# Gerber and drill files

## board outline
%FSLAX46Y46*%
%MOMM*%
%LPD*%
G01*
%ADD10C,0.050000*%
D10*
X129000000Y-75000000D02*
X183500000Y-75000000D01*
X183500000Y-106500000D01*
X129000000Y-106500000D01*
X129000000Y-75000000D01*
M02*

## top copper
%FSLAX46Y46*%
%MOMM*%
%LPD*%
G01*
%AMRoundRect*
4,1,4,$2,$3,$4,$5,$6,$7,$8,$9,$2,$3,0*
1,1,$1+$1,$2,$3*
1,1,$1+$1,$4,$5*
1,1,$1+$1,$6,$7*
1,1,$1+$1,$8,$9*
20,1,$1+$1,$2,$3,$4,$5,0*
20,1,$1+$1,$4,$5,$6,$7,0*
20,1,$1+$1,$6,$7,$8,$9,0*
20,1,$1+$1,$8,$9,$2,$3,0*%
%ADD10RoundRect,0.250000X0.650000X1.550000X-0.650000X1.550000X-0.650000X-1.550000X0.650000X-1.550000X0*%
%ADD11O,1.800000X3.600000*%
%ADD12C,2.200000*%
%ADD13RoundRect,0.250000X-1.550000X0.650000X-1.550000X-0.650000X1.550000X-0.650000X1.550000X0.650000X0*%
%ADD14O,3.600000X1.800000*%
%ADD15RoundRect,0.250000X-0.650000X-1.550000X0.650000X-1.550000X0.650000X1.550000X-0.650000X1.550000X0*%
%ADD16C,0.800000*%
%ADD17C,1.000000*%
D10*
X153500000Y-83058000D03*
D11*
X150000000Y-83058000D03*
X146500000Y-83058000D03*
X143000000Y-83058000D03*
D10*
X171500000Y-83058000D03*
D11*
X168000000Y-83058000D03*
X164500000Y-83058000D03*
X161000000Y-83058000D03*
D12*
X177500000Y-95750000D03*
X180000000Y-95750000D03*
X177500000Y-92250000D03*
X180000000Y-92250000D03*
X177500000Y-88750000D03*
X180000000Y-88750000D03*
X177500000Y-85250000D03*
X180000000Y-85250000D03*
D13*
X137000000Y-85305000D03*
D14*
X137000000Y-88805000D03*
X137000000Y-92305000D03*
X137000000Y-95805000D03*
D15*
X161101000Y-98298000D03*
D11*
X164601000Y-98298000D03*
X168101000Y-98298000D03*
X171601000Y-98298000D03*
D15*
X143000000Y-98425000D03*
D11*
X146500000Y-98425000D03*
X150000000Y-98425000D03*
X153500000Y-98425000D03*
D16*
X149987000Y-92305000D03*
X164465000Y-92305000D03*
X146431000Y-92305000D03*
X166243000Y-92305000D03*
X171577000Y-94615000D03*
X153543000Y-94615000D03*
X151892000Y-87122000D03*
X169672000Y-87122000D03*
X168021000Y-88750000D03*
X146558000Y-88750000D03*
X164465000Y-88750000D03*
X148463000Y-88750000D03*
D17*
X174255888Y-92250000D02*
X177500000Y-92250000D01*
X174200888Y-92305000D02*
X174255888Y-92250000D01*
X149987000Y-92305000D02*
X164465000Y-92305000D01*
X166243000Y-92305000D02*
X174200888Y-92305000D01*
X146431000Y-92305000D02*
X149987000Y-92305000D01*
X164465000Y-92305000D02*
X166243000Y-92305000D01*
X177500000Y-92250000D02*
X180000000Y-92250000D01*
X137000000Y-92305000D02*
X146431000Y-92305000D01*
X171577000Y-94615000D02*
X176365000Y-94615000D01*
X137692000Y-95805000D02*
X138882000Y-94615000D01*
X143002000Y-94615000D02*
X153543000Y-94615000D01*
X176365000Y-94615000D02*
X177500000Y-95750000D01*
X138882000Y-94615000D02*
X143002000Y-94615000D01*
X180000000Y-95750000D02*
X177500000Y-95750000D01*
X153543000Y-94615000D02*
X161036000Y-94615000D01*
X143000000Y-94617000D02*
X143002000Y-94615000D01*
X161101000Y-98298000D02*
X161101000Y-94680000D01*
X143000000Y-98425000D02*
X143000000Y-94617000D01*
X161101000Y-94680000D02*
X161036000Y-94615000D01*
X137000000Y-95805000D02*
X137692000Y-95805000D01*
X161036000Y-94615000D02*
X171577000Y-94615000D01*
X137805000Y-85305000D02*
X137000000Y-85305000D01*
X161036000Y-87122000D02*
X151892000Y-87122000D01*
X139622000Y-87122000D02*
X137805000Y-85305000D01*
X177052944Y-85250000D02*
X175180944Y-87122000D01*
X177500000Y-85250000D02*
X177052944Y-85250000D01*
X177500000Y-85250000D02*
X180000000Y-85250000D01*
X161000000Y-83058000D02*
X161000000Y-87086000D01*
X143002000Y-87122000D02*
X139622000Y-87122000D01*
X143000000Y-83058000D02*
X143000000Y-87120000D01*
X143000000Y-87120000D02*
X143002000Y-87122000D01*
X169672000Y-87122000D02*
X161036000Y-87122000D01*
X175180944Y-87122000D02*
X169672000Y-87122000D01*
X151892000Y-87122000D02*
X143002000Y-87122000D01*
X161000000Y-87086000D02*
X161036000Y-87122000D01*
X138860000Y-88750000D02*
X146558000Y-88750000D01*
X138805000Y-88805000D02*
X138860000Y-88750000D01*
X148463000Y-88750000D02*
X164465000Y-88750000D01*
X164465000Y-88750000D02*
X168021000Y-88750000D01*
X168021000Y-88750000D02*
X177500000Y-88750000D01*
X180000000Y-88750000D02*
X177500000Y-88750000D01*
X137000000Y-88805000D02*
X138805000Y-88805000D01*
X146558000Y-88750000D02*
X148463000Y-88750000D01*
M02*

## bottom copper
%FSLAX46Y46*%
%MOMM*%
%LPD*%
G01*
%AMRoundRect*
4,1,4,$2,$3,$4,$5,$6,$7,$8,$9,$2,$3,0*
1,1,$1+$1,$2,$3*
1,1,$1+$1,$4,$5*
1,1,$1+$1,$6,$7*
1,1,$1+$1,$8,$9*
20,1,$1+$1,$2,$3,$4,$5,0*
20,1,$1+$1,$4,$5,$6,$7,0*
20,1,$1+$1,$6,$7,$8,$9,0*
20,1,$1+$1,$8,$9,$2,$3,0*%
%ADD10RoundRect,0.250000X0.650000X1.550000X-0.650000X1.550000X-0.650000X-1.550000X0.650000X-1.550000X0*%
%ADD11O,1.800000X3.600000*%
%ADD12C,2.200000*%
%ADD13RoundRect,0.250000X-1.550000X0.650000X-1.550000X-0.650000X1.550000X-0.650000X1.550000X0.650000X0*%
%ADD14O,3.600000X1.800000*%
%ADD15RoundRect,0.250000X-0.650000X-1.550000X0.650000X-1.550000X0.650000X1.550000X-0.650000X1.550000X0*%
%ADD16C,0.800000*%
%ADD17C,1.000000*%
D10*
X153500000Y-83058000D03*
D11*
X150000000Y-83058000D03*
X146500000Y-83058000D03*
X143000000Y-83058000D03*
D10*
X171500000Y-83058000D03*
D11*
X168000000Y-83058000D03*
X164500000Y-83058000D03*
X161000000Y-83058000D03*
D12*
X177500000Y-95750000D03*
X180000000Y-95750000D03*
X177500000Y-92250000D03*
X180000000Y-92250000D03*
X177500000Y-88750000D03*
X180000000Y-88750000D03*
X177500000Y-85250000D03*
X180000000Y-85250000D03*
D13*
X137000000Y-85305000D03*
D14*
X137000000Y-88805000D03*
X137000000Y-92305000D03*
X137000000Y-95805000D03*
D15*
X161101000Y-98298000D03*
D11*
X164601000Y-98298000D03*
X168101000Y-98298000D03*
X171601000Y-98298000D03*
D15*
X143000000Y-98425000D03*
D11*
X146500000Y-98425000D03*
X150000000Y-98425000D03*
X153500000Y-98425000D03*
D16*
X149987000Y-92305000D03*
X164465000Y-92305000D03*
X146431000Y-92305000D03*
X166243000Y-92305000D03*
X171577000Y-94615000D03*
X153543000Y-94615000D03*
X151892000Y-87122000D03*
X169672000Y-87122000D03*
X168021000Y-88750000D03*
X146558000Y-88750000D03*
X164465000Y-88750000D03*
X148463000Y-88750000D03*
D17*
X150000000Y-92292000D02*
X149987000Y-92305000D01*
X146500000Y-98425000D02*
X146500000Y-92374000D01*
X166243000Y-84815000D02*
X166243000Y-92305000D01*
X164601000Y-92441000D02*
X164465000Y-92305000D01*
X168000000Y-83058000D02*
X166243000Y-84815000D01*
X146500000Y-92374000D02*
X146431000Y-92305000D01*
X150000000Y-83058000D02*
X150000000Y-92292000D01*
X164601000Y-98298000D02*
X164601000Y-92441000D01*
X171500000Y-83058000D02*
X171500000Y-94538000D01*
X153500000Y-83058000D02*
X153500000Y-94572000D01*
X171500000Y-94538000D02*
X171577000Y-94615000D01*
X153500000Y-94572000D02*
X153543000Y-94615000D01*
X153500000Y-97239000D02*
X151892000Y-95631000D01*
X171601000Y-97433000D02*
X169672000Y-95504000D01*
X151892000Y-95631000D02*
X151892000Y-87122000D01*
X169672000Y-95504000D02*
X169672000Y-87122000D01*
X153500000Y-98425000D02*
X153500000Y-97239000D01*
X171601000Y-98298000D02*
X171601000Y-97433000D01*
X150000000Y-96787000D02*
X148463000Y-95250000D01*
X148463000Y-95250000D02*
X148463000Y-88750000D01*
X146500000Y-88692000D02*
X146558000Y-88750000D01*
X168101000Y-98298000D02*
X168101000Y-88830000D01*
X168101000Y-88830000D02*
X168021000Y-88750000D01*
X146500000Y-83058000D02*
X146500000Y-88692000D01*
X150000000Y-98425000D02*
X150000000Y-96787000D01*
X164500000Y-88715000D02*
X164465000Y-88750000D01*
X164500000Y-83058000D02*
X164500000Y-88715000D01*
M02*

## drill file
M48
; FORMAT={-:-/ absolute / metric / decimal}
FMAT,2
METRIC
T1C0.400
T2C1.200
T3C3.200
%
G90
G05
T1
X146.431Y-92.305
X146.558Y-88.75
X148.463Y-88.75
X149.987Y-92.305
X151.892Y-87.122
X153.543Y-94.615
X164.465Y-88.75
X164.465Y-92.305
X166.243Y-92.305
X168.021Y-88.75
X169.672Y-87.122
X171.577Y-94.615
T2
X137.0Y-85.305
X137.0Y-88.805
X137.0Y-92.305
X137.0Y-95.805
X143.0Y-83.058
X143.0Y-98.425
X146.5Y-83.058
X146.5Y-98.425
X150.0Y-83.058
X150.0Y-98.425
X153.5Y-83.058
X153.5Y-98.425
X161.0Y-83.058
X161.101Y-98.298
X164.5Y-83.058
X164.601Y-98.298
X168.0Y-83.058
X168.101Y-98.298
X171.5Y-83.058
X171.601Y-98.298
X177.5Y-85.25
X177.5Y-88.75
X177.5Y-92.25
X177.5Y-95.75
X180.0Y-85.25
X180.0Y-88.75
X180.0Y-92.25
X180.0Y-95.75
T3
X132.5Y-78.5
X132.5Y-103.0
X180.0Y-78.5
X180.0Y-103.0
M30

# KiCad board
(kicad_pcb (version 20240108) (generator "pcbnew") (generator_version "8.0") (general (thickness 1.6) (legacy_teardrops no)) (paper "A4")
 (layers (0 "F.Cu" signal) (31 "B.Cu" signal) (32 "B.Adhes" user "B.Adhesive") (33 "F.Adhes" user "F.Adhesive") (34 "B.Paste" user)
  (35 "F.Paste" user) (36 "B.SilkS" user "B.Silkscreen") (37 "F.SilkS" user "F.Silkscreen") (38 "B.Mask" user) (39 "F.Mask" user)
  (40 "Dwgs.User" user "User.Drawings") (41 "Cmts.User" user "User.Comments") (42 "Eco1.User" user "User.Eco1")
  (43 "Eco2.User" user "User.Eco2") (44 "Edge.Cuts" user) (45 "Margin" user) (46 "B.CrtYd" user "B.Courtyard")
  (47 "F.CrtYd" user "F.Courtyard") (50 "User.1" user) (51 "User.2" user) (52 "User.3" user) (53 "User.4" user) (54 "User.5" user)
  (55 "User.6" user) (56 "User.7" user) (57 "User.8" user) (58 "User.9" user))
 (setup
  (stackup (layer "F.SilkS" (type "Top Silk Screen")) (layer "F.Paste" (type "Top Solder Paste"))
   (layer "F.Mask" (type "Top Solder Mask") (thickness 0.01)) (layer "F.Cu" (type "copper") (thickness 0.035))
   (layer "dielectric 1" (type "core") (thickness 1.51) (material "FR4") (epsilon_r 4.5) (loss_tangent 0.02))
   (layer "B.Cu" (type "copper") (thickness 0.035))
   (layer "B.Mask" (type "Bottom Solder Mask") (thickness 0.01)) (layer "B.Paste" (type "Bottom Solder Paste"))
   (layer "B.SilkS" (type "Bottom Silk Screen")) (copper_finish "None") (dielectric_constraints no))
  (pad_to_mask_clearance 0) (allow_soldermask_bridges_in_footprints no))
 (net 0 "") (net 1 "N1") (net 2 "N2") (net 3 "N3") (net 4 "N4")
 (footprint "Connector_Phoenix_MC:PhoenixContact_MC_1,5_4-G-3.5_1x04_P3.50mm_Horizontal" (layer "F.Cu") (at 153.5 83.058 180)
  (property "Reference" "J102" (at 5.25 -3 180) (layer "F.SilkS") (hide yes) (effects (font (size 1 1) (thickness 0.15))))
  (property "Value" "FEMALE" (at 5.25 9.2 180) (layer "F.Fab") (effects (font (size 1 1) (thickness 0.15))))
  (pad "1" thru_hole roundrect (at 0 0 180) (size 1.8 3.6) (drill 1.2) (layers "*.Cu" "*.Mask") (remove_unused_layers no)
   (roundrect_rratio 0.138889) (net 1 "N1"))
  (pad "2" thru_hole oval (at 3.5 0 180) (size 1.8 3.6) (drill 1.2) (layers "*.Cu" "*.Mask") (remove_unused_layers no) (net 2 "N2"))
  (pad "3" thru_hole oval (at 7 0 180) (size 1.8 3.6) (drill 1.2) (layers "*.Cu" "*.Mask") (remove_unused_layers no) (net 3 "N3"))
  (pad "4" thru_hole oval (at 10.5 0 180) (size 1.8 3.6) (drill 1.2) (layers "*.Cu" "*.Mask") (remove_unused_layers no) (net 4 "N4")))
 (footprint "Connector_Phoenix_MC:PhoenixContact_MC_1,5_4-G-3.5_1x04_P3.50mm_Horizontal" (layer "F.Cu") (at 171.5 83.058 180)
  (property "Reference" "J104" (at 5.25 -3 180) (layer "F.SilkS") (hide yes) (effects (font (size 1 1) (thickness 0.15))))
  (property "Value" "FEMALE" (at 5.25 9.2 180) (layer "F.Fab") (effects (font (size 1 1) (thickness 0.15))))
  (pad "1" thru_hole roundrect (at 0 0 180) (size 1.8 3.6) (drill 1.2) (layers "*.Cu" "*.Mask") (remove_unused_layers no)
   (roundrect_rratio 0.138889) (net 1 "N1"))
  (pad "2" thru_hole oval (at 3.5 0 180) (size 1.8 3.6) (drill 1.2) (layers "*.Cu" "*.Mask") (remove_unused_layers no) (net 2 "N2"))
  (pad "3" thru_hole oval (at 7 0 180) (size 1.8 3.6) (drill 1.2) (layers "*.Cu" "*.Mask") (remove_unused_layers no) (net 3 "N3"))
  (pad "4" thru_hole oval (at 10.5 0 180) (size 1.8 3.6) (drill 1.2) (layers "*.Cu" "*.Mask") (remove_unused_layers no) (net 4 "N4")))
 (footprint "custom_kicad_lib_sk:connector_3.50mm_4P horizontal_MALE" (layer "F.Cu") (at 177.5 90.5 90)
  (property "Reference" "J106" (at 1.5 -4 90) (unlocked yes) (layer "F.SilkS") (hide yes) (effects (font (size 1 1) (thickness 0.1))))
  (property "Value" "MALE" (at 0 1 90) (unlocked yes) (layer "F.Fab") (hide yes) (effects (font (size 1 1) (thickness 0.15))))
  (pad "1" thru_hole circle (at -5.25 0 90) (size 2.2 2.2) (drill 1.2) (layers "*.Cu" "*.Mask") (remove_unused_layers no) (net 1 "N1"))
  (pad "1" thru_hole circle (at -5.25 2.5 90) (size 2.2 2.2) (drill 1.2) (layers "*.Cu" "*.Mask") (remove_unused_layers no) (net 1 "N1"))
  (pad "2" thru_hole circle (at -1.75 0 90) (size 2.2 2.2) (drill 1.2) (layers "*.Cu" "*.Mask") (remove_unused_layers no) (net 2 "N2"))
  (pad "2" thru_hole circle (at -1.75 2.5 90) (size 2.2 2.2) (drill 1.2) (layers "*.Cu" "*.Mask") (remove_unused_layers no) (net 2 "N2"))
  (pad "3" thru_hole circle (at 1.75 0 90) (size 2.2 2.2) (drill 1.2) (layers "*.Cu" "*.Mask") (remove_unused_layers no) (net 3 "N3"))
  (pad "3" thru_hole circle (at 1.75 2.5 90) (size 2.2 2.2) (drill 1.2) (layers "*.Cu" "*.Mask") (remove_unused_layers no) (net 3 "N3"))
  (pad "4" thru_hole circle (at 5.25 0 90) (size 2.2 2.2) (drill 1.2) (layers "*.Cu" "*.Mask") (remove_unused_layers no) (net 4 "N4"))
  (pad "4" thru_hole circle (at 5.25 2.5 90) (size 2.2 2.2) (drill 1.2) (layers "*.Cu" "*.Mask") (remove_unused_layers no) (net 4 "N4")))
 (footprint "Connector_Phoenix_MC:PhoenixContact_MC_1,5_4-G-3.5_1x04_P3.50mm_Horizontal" (layer "F.Cu") (at 137 85.305 -90)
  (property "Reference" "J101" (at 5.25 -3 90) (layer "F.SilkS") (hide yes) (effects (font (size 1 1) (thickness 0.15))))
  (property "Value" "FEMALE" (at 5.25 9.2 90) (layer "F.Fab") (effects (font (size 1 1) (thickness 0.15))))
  (pad "1" thru_hole roundrect (at 0 0 270) (size 1.8 3.6) (drill 1.2) (layers "*.Cu" "*.Mask") (remove_unused_layers no)
   (roundrect_rratio 0.138889) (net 4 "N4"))
  (pad "2" thru_hole oval (at 3.5 0 270) (size 1.8 3.6) (drill 1.2) (layers "*.Cu" "*.Mask") (remove_unused_layers no) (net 3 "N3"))
  (pad "3" thru_hole oval (at 7 0 270) (size 1.8 3.6) (drill 1.2) (layers "*.Cu" "*.Mask") (remove_unused_layers no) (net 2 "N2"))
  (pad "4" thru_hole oval (at 10.5 0 270) (size 1.8 3.6) (drill 1.2) (layers "*.Cu" "*.Mask") (remove_unused_layers no) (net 1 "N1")))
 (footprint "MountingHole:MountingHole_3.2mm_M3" (layer "F.Cu") (at 132.5 103)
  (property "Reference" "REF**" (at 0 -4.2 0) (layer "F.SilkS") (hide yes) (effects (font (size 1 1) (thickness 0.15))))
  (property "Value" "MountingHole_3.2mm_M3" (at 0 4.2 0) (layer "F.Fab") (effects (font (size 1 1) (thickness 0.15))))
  (pad "" np_thru_hole circle (at 0 0) (size 3.2 3.2) (drill 3.2) (layers "F&B.Cu" "*.Mask")))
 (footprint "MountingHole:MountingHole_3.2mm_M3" (layer "F.Cu") (at 180 78.5)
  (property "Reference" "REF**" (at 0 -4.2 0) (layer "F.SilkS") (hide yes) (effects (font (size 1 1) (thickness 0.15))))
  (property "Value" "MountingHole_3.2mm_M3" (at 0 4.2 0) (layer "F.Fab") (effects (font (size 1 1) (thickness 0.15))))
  (pad "" np_thru_hole circle (at 0 0) (size 3.2 3.2) (drill 3.2) (layers "F&B.Cu" "*.Mask")))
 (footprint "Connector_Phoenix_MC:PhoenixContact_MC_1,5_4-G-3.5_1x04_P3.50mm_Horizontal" (layer "F.Cu") (at 161.101 98.298)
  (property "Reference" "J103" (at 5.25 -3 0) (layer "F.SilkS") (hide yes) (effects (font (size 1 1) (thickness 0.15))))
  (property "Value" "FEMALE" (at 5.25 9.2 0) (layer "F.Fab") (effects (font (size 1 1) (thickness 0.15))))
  (pad "1" thru_hole roundrect (at 0 0) (size 1.8 3.6) (drill 1.2) (layers "*.Cu" "*.Mask") (remove_unused_layers no)
   (roundrect_rratio 0.138889) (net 1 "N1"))
  (pad "2" thru_hole oval (at 3.5 0) (size 1.8 3.6) (drill 1.2) (layers "*.Cu" "*.Mask") (remove_unused_layers no) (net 2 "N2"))
  (pad "3" thru_hole oval (at 7 0) (size 1.8 3.6) (drill 1.2) (layers "*.Cu" "*.Mask") (remove_unused_layers no) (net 3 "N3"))
  (pad "4" thru_hole oval (at 10.5 0) (size 1.8 3.6) (drill 1.2) (layers "*.Cu" "*.Mask") (remove_unused_layers no) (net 4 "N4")))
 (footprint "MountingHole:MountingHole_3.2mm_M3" (layer "F.Cu") (at 180 103)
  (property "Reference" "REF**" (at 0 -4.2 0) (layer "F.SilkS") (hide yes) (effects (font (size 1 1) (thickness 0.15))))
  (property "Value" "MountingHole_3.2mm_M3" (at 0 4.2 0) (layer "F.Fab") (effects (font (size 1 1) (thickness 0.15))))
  (pad "" np_thru_hole circle (at 0 0) (size 3.2 3.2) (drill 3.2) (layers "F&B.Cu" "*.Mask")))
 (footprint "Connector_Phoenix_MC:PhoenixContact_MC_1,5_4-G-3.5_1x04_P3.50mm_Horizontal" (layer "F.Cu") (at 143 98.425)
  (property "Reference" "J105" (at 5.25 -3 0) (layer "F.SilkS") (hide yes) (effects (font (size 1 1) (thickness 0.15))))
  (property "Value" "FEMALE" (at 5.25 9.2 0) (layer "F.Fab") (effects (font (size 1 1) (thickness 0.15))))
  (pad "1" thru_hole roundrect (at 0 0) (size 1.8 3.6) (drill 1.2) (layers "*.Cu" "*.Mask") (remove_unused_layers no)
   (roundrect_rratio 0.138889) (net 1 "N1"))
  (pad "2" thru_hole oval (at 3.5 0) (size 1.8 3.6) (drill 1.2) (layers "*.Cu" "*.Mask") (remove_unused_layers no) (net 2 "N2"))
  (pad "3" thru_hole oval (at 7 0) (size 1.8 3.6) (drill 1.2) (layers "*.Cu" "*.Mask") (remove_unused_layers no) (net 3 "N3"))
  (pad "4" thru_hole oval (at 10.5 0) (size 1.8 3.6) (drill 1.2) (layers "*.Cu" "*.Mask") (remove_unused_layers no) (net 4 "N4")))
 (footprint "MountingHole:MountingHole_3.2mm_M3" (layer "F.Cu") (at 132.5 78.5)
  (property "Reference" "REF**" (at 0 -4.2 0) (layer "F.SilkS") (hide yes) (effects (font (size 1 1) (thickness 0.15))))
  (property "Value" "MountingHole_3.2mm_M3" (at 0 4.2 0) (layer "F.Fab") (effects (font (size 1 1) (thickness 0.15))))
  (pad "" np_thru_hole circle (at 0 0) (size 3.2 3.2) (drill 3.2) (layers "*.Cu" "*.Mask")))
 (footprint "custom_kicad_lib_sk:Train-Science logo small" (layer "B.Cu") (at 157.099 90.932 180)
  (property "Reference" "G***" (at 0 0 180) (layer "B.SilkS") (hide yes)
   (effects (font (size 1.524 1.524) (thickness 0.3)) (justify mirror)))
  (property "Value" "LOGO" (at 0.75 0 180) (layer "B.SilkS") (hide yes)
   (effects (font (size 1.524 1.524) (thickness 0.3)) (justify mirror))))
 (gr_rect (start 129 75) (end 183.5 106.5) (stroke (width 0.05) (type default)) (fill none) (layer "Edge.Cuts"))
 (segment (start 174.255888 92.25) (end 177.5 92.25) (width 1) (layer "F.Cu") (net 2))
 (segment (start 174.200888 92.305) (end 174.255888 92.25) (width 1) (layer "F.Cu") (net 2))
 (segment (start 149.987 92.305) (end 164.465 92.305) (width 1) (layer "F.Cu") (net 2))
 (segment (start 166.243 92.305) (end 174.200888 92.305) (width 1) (layer "F.Cu") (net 2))
 (segment (start 146.431 92.305) (end 149.987 92.305) (width 1) (layer "F.Cu") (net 2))
 (segment (start 164.465 92.305) (end 166.243 92.305) (width 1) (layer "F.Cu") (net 2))
 (segment (start 177.5 92.25) (end 180 92.25) (width 1) (layer "F.Cu") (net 2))
 (segment (start 137 92.305) (end 146.431 92.305) (width 1) (layer "F.Cu") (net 2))
 (via (at 149.987 92.305) (size 0.8) (drill 0.4) (layers "F.Cu" "B.Cu") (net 2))
 (via (at 164.465 92.305) (size 0.8) (drill 0.4) (layers "F.Cu" "B.Cu") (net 2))
 (via (at 146.431 92.305) (size 0.8) (drill 0.4) (layers "F.Cu" "B.Cu") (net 2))
 (via (at 166.243 92.305) (size 0.8) (drill 0.4) (layers "F.Cu" "B.Cu") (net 2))
 (segment (start 150 92.292) (end 149.987 92.305) (width 1) (layer "B.Cu") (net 2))
 (segment (start 146.5 98.425) (end 146.5 92.374) (width 1) (layer "B.Cu") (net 2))
 (segment (start 166.243 84.815) (end 166.243 92.305) (width 1) (layer "B.Cu") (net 2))
 (segment (start 164.601 92.441) (end 164.465 92.305) (width 1) (layer "B.Cu") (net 2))
 (segment (start 168 83.058) (end 166.243 84.815) (width 1) (layer "B.Cu") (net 2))
 (segment (start 146.5 92.374) (end 146.431 92.305) (width 1) (layer "B.Cu") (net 2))
 (segment (start 150 83.058) (end 150 92.292) (width 1) (layer "B.Cu") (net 2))
 (segment (start 164.601 98.298) (end 164.601 92.441) (width 1) (layer "B.Cu") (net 2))
 (segment (start 171.577 94.615) (end 176.365 94.615) (width 1) (layer "F.Cu") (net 1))
 (segment (start 137.692 95.805) (end 138.882 94.615) (width 1) (layer "F.Cu") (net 1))
 (segment (start 143.002 94.615) (end 153.543 94.615) (width 1) (layer "F.Cu") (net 1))
 (segment (start 176.365 94.615) (end 177.5 95.75) (width 1) (layer "F.Cu") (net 1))
 (segment (start 138.882 94.615) (end 143.002 94.615) (width 1) (layer "F.Cu") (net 1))
 (segment (start 180 95.75) (end 177.5 95.75) (width 1) (layer "F.Cu") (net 1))
 (segment (start 153.543 94.615) (end 161.036 94.615) (width 1) (layer "F.Cu") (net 1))
 (segment (start 143 94.617) (end 143.002 94.615) (width 1) (layer "F.Cu") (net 1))
 (segment (start 161.101 98.298) (end 161.101 94.68) (width 1) (layer "F.Cu") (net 1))
 (segment (start 143 98.425) (end 143 94.617) (width 1) (layer "F.Cu") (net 1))
 (segment (start 161.101 94.68) (end 161.036 94.615) (width 1) (layer "F.Cu") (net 1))
 (segment (start 137 95.805) (end 137.692 95.805) (width 1) (layer "F.Cu") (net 1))
 (segment (start 161.036 94.615) (end 171.577 94.615) (width 1) (layer "F.Cu") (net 1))
 (via (at 171.577 94.615) (size 0.8) (drill 0.4) (layers "F.Cu" "B.Cu") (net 1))
 (via (at 153.543 94.615) (size 0.8) (drill 0.4) (layers "F.Cu" "B.Cu") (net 1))
 (segment (start 171.5 83.058) (end 171.5 94.538) (width 1) (layer "B.Cu") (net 1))
 (segment (start 153.5 83.058) (end 153.5 94.572) (width 1) (layer "B.Cu") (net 1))
 (segment (start 171.5 94.538) (end 171.577 94.615) (width 1) (layer "B.Cu") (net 1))
 (segment (start 153.5 94.572) (end 153.543 94.615) (width 1) (layer "B.Cu") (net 1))
 (segment (start 137.805 85.305) (end 137 85.305) (width 1) (layer "F.Cu") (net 4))
 (segment (start 161.036 87.122) (end 151.892 87.122) (width 1) (layer "F.Cu") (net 4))
 (segment (start 139.622 87.122) (end 137.805 85.305) (width 1) (layer "F.Cu") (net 4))
 (segment (start 177.052944 85.25) (end 175.180944 87.122) (width 1) (layer "F.Cu") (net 4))
 (segment (start 177.5 85.25) (end 177.052944 85.25) (width 1) (layer "F.Cu") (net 4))
 (segment (start 177.5 85.25) (end 180 85.25) (width 1) (layer "F.Cu") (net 4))
 (segment (start 161 83.058) (end 161 87.086) (width 1) (layer "F.Cu") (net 4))
 (segment (start 143.002 87.122) (end 139.622 87.122) (width 1) (layer "F.Cu") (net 4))
 (segment (start 143 83.058) (end 143 87.12) (width 1) (layer "F.Cu") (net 4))
 (segment (start 143 87.12) (end 143.002 87.122) (width 1) (layer "F.Cu") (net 4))
 (segment (start 169.672 87.122) (end 161.036 87.122) (width 1) (layer "F.Cu") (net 4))
 (segment (start 175.180944 87.122) (end 169.672 87.122) (width 1) (layer "F.Cu") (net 4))
 (segment (start 151.892 87.122) (end 143.002 87.122) (width 1) (layer "F.Cu") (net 4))
 (segment (start 161 87.086) (end 161.036 87.122) (width 1) (layer "F.Cu") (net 4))
 (via (at 151.892 87.122) (size 0.8) (drill 0.4) (layers "F.Cu" "B.Cu") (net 4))
 (via (at 169.672 87.122) (size 0.8) (drill 0.4) (layers "F.Cu" "B.Cu") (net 4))
 (segment (start 153.5 97.239) (end 151.892 95.631) (width 1) (layer "B.Cu") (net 4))
 (segment (start 171.601 97.433) (end 169.672 95.504) (width 1) (layer "B.Cu") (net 4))
 (segment (start 151.892 95.631) (end 151.892 87.122) (width 1) (layer "B.Cu") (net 4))
 (segment (start 169.672 95.504) (end 169.672 87.122) (width 1) (layer "B.Cu") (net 4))
 (segment (start 153.5 98.425) (end 153.5 97.239) (width 1) (layer "B.Cu") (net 4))
 (segment (start 171.601 98.298) (end 171.601 97.433) (width 1) (layer "B.Cu") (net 4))
 (segment (start 138.86 88.75) (end 146.558 88.75) (width 1) (layer "F.Cu") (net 3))
 (segment (start 138.805 88.805) (end 138.86 88.75) (width 1) (layer "F.Cu") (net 3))
 (segment (start 148.463 88.75) (end 164.465 88.75) (width 1) (layer "F.Cu") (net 3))
 (segment (start 164.465 88.75) (end 168.021 88.75) (width 1) (layer "F.Cu") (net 3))
 (segment (start 168.021 88.75) (end 177.5 88.75) (width 1) (layer "F.Cu") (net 3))
 (segment (start 180 88.75) (end 177.5 88.75) (width 1) (layer "F.Cu") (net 3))
 (segment (start 137 88.805) (end 138.805 88.805) (width 1) (layer "F.Cu") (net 3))
 (segment (start 146.558 88.75) (end 148.463 88.75) (width 1) (layer "F.Cu") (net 3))
 (via (at 168.021 88.75) (size 0.8) (drill 0.4) (layers "F.Cu" "B.Cu") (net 3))
 (via (at 146.558 88.75) (size 0.8) (drill 0.4) (layers "F.Cu" "B.Cu") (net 3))
 (via (at 164.465 88.75) (size 0.8) (drill 0.4) (layers "F.Cu" "B.Cu") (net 3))
 (via (at 148.463 88.75) (size 0.8) (drill 0.4) (layers "F.Cu" "B.Cu") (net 3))
 (segment (start 150 96.787) (end 148.463 95.25) (width 1) (layer "B.Cu") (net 3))
 (segment (start 148.463 95.25) (end 148.463 88.75) (width 1) (layer "B.Cu") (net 3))
 (segment (start 146.5 88.692) (end 146.558 88.75) (width 1) (layer "B.Cu") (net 3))
 (segment (start 168.101 98.298) (end 168.101 88.83) (width 1) (layer "B.Cu") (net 3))
 (segment (start 168.101 88.83) (end 168.021 88.75) (width 1) (layer "B.Cu") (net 3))
 (segment (start 146.5 83.058) (end 146.5 88.692) (width 1) (layer "B.Cu") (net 3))
 (segment (start 150 98.425) (end 150 96.787) (width 1) (layer "B.Cu") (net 3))
 (segment (start 164.5 88.715) (end 164.465 88.75) (width 1) (layer "B.Cu") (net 3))
 (segment (start 164.5 83.058) (end 164.5 88.715) (width 1) (layer "B.Cu") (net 3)))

